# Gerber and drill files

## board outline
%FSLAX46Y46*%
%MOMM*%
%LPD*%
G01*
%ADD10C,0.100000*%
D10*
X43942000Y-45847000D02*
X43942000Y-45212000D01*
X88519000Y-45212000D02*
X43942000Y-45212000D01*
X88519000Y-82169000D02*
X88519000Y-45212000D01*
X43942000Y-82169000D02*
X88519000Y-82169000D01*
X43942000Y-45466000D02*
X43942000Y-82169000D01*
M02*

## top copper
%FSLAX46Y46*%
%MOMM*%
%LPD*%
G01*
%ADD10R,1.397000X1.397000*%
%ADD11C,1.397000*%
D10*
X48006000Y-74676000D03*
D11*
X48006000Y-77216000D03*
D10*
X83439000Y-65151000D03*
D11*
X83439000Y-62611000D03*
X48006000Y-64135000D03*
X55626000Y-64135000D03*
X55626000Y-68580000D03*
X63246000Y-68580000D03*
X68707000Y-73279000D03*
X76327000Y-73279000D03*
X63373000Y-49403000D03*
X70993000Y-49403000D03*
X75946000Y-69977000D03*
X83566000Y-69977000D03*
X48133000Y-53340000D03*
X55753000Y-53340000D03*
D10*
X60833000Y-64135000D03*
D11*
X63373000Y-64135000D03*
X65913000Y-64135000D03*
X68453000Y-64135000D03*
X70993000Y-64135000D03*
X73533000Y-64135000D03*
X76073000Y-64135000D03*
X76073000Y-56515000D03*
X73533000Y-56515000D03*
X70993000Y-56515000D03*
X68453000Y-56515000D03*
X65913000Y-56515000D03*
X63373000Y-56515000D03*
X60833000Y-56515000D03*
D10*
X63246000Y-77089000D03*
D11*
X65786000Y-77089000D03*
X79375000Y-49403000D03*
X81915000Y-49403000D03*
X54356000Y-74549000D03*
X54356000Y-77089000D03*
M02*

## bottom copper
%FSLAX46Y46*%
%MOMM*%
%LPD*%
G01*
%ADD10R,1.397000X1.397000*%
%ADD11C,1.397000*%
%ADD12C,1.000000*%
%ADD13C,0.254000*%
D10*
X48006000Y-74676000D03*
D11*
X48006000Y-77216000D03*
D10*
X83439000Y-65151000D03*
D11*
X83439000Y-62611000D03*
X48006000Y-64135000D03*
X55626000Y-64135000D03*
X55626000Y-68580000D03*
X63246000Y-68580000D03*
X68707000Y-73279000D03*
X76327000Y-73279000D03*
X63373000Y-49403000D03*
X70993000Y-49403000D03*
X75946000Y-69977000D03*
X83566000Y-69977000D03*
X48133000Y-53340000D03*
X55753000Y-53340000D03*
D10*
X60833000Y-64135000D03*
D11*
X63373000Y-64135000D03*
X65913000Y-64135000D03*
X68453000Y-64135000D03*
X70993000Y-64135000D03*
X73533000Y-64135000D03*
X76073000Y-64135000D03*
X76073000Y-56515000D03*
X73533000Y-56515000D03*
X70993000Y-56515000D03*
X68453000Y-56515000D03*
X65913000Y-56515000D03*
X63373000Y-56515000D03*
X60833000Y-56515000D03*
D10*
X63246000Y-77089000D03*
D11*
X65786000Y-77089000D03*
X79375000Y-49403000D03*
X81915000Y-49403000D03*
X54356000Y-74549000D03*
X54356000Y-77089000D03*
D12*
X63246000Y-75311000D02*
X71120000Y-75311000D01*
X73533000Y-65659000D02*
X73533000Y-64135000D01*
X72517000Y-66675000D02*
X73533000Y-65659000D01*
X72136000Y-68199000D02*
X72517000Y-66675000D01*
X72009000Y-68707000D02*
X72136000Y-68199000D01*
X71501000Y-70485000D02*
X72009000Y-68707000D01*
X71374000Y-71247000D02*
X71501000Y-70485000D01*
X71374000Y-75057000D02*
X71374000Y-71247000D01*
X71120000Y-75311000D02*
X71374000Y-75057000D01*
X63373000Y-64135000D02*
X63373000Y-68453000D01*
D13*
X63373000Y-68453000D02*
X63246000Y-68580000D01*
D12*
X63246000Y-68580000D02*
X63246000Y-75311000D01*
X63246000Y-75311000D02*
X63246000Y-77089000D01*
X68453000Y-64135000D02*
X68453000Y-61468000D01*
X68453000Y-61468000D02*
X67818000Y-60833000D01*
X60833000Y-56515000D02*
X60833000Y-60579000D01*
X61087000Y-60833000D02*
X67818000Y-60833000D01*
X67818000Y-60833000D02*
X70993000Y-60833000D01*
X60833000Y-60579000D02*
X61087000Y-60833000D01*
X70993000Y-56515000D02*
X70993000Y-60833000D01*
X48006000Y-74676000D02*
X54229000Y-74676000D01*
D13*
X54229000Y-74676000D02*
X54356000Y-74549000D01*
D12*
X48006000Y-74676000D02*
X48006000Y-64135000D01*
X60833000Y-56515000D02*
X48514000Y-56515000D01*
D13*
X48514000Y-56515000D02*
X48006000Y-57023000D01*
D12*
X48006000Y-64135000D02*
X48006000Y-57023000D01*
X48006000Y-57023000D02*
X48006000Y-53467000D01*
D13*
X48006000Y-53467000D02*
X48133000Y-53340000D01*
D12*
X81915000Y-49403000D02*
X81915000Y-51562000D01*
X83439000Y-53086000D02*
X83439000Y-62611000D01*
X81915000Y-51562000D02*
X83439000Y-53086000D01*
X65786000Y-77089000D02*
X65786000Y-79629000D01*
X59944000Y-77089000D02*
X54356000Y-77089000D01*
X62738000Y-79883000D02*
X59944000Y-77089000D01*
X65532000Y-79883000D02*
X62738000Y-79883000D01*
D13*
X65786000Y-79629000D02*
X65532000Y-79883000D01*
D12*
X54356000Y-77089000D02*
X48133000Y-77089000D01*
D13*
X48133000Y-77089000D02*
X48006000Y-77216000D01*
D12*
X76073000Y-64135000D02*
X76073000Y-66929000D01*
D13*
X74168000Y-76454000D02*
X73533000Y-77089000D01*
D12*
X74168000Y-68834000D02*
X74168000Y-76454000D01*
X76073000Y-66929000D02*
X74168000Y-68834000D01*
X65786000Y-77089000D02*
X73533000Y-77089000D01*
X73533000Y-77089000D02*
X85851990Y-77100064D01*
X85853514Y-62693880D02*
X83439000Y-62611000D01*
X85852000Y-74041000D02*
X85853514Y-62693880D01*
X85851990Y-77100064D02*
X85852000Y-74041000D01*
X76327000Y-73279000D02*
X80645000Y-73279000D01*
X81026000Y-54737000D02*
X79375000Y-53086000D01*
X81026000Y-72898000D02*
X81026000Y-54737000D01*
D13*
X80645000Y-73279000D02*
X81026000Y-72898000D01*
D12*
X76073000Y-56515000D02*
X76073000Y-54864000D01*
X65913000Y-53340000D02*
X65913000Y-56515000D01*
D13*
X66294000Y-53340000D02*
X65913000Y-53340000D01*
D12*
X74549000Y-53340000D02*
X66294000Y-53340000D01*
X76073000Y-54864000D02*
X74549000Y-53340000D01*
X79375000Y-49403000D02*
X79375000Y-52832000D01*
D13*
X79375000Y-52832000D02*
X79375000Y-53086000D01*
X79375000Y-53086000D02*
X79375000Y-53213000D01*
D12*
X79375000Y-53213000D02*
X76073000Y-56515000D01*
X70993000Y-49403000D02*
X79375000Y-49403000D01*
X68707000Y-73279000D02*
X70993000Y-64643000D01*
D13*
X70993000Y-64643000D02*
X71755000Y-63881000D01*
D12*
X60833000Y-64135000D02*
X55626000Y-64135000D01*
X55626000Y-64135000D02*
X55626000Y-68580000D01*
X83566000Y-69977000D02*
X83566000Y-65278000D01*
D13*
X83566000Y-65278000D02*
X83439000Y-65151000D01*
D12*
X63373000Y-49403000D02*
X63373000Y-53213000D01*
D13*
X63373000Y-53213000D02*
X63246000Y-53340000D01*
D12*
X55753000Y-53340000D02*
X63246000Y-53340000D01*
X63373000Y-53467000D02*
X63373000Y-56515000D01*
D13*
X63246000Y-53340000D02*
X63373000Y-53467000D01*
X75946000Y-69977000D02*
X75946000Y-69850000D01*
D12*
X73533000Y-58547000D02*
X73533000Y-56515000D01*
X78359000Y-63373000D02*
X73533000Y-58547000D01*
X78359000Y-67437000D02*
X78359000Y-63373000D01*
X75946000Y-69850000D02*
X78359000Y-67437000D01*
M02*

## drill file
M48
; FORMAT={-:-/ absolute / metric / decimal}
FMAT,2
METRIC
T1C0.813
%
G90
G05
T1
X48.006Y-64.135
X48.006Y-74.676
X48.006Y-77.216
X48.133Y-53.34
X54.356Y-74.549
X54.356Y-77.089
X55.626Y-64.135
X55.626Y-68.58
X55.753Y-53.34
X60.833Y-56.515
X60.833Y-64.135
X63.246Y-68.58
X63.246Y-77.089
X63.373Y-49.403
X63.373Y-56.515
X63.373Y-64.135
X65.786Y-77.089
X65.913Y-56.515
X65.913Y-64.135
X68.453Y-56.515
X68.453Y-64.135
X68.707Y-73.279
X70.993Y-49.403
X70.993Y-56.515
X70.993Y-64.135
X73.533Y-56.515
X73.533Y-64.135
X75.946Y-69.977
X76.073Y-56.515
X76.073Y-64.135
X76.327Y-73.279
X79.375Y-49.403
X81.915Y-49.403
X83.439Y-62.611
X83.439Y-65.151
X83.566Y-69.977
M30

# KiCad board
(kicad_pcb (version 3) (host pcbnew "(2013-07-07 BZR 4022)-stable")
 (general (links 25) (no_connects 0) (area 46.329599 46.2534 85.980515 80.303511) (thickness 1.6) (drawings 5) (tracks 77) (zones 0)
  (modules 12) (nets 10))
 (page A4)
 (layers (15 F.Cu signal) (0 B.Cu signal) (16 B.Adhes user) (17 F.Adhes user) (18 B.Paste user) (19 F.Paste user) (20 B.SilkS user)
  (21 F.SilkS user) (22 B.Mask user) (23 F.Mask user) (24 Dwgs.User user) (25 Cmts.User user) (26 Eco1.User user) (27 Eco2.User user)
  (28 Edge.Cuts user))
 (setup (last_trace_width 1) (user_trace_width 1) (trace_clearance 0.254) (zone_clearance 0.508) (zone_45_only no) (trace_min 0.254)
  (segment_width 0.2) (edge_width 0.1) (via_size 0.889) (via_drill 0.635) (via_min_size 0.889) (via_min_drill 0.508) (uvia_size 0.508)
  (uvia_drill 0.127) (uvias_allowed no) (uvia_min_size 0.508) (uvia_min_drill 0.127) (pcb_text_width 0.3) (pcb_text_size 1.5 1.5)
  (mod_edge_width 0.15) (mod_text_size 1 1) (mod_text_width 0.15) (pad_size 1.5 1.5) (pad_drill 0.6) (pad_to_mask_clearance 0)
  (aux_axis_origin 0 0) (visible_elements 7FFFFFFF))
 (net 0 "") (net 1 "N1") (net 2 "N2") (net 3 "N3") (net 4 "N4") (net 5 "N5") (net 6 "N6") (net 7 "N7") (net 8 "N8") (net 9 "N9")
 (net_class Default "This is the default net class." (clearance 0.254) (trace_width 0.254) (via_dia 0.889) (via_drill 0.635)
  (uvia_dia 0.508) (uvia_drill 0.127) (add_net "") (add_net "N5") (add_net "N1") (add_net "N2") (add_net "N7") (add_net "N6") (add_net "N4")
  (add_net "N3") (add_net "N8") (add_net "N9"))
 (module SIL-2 (layer F.Cu) (at 48.006 75.946 270)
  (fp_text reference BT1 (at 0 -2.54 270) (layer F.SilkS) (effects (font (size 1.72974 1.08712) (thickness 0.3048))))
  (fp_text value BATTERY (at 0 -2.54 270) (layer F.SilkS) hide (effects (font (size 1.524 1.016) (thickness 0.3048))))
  (pad 1 thru_hole rect (at -1.27 0 270) (size 1.397 1.397) (drill 0.8128) (layers *.Cu *.Mask F.SilkS) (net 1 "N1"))
  (pad 2 thru_hole circle (at 1.27 0 270) (size 1.397 1.397) (drill 0.8128) (layers *.Cu *.Mask F.SilkS) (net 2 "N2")))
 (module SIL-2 (layer F.Cu) (at 83.439 63.881 90)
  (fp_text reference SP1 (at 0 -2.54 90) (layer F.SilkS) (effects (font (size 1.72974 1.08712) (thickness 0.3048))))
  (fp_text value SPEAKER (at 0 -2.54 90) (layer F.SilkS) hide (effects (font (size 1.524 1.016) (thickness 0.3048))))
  (pad 1 thru_hole rect (at -1.27 0 90) (size 1.397 1.397) (drill 0.8128) (layers *.Cu *.Mask F.SilkS) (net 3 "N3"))
  (pad 2 thru_hole circle (at 1.27 0 90) (size 1.397 1.397) (drill 0.8128) (layers *.Cu *.Mask F.SilkS) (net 2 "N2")))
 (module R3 (layer F.Cu) (at 51.816 64.135) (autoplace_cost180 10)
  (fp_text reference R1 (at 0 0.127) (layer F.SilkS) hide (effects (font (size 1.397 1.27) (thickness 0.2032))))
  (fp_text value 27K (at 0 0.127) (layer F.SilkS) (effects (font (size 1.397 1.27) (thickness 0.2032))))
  (pad 1 thru_hole circle (at -3.81 0) (size 1.397 1.397) (drill 0.8128) (layers *.Cu *.Mask F.SilkS) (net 1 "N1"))
  (pad 2 thru_hole circle (at 3.81 0) (size 1.397 1.397) (drill 0.8128) (layers *.Cu *.Mask F.SilkS) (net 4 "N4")))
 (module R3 (layer F.Cu) (at 59.436 68.58) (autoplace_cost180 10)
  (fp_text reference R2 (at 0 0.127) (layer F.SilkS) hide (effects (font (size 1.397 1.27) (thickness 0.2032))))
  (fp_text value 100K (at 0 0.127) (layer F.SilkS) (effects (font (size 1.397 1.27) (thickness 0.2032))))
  (pad 1 thru_hole circle (at -3.81 0) (size 1.397 1.397) (drill 0.8128) (layers *.Cu *.Mask F.SilkS) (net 4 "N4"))
  (pad 2 thru_hole circle (at 3.81 0) (size 1.397 1.397) (drill 0.8128) (layers *.Cu *.Mask F.SilkS) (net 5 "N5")))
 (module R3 (layer F.Cu) (at 72.517 73.279) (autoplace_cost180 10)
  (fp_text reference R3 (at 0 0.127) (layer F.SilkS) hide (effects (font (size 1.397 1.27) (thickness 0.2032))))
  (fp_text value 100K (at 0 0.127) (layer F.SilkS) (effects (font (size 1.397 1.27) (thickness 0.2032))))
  (pad 1 thru_hole circle (at -3.81 0) (size 1.397 1.397) (drill 0.8128) (layers *.Cu *.Mask F.SilkS) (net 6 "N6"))
  (pad 2 thru_hole circle (at 3.81 0) (size 1.397 1.397) (drill 0.8128) (layers *.Cu *.Mask F.SilkS) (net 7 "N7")))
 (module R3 (layer F.Cu) (at 67.183 49.403) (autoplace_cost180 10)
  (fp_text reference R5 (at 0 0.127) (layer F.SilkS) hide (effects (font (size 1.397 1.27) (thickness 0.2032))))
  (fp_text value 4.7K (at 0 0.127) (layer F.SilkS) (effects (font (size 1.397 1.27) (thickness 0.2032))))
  (pad 1 thru_hole circle (at -3.81 0) (size 1.397 1.397) (drill 0.8128) (layers *.Cu *.Mask F.SilkS) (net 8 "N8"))
  (pad 2 thru_hole circle (at 3.81 0) (size 1.397 1.397) (drill 0.8128) (layers *.Cu *.Mask F.SilkS) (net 7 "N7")))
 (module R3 (layer F.Cu) (at 79.756 69.977) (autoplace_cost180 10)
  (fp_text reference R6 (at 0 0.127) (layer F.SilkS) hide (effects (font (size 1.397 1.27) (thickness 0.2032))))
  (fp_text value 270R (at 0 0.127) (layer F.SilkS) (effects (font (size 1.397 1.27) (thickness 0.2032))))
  (pad 1 thru_hole circle (at -3.81 0) (size 1.397 1.397) (drill 0.8128) (layers *.Cu *.Mask F.SilkS) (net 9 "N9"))
  (pad 2 thru_hole circle (at 3.81 0) (size 1.397 1.397) (drill 0.8128) (layers *.Cu *.Mask F.SilkS) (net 3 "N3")))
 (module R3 (layer F.Cu) (at 51.943 53.34) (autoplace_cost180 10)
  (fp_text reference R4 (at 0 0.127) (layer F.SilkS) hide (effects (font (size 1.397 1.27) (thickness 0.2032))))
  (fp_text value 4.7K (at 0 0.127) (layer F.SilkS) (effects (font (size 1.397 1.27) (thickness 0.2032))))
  (pad 1 thru_hole circle (at -3.81 0) (size 1.397 1.397) (drill 0.8128) (layers *.Cu *.Mask F.SilkS) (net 1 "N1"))
  (pad 2 thru_hole circle (at 3.81 0) (size 1.397 1.397) (drill 0.8128) (layers *.Cu *.Mask F.SilkS) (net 8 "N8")))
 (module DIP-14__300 (layer F.Cu) (at 68.453 60.325)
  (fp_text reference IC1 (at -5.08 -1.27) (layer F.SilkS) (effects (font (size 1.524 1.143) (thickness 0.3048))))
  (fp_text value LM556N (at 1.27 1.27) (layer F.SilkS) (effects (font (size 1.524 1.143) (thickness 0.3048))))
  (pad 1 thru_hole rect (at -7.62 3.81) (size 1.397 1.397) (drill 0.8128) (layers *.Cu *.Mask F.SilkS) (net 4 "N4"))
  (pad 2 thru_hole circle (at -5.08 3.81) (size 1.397 1.397) (drill 0.8128) (layers *.Cu *.Mask F.SilkS) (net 5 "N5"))
  (pad 3 thru_hole circle (at -2.54 3.81) (size 1.397 1.397) (drill 0.8128) (layers *.Cu *.Mask F.SilkS))
  (pad 4 thru_hole circle (at 0 3.81) (size 1.397 1.397) (drill 0.8128) (layers *.Cu *.Mask F.SilkS) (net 1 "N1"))
  (pad 5 thru_hole circle (at 2.54 3.81) (size 1.397 1.397) (drill 0.8128) (layers *.Cu *.Mask F.SilkS) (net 6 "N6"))
  (pad 6 thru_hole circle (at 5.08 3.81) (size 1.397 1.397) (drill 0.8128) (layers *.Cu *.Mask F.SilkS) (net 5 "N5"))
  (pad 7 thru_hole circle (at 7.62 3.81) (size 1.397 1.397) (drill 0.8128) (layers *.Cu *.Mask F.SilkS) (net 2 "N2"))
  (pad 8 thru_hole circle (at 7.62 -3.81) (size 1.397 1.397) (drill 0.8128) (layers *.Cu *.Mask F.SilkS) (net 7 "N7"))
  (pad 9 thru_hole circle (at 5.08 -3.81) (size 1.397 1.397) (drill 0.8128) (layers *.Cu *.Mask F.SilkS) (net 9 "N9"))
  (pad 10 thru_hole circle (at 2.54 -3.81) (size 1.397 1.397) (drill 0.8128) (layers *.Cu *.Mask F.SilkS) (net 1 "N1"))
  (pad 11 thru_hole circle (at 0 -3.81) (size 1.397 1.397) (drill 0.8128) (layers *.Cu *.Mask F.SilkS))
  (pad 12 thru_hole circle (at -2.54 -3.81) (size 1.397 1.397) (drill 0.8128) (layers *.Cu *.Mask F.SilkS) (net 7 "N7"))
  (pad 13 thru_hole circle (at -5.08 -3.81) (size 1.397 1.397) (drill 0.8128) (layers *.Cu *.Mask F.SilkS) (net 8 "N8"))
  (pad 14 thru_hole circle (at -7.62 -3.81) (size 1.397 1.397) (drill 0.8128) (layers *.Cu *.Mask F.SilkS) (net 1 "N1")))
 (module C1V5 (layer F.Cu) (at 64.516 77.089)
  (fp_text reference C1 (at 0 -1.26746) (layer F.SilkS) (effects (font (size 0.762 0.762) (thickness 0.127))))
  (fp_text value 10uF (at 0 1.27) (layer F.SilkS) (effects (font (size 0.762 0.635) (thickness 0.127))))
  (pad 1 thru_hole rect (at -1.27 0) (size 1.397 1.397) (drill 0.8128) (layers *.Cu *.Mask F.SilkS) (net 5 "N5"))
  (pad 2 thru_hole circle (at 1.27 0) (size 1.397 1.397) (drill 0.8128) (layers *.Cu *.Mask F.SilkS) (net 2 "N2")))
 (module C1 (layer F.Cu) (at 80.645 49.403)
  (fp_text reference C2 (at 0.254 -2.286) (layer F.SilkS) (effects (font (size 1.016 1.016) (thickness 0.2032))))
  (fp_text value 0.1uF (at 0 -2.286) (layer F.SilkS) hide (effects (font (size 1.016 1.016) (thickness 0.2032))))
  (pad 1 thru_hole circle (at -1.27 0) (size 1.397 1.397) (drill 0.8128) (layers *.Cu *.Mask F.SilkS) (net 7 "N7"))
  (pad 2 thru_hole circle (at 1.27 0) (size 1.397 1.397) (drill 0.8128) (layers *.Cu *.Mask F.SilkS) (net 2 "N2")))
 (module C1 (layer F.Cu) (at 54.356 75.819 270)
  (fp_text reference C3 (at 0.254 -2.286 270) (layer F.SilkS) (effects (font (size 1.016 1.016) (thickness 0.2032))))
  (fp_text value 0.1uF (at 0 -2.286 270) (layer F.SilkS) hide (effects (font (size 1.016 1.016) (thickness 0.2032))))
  (pad 1 thru_hole circle (at -1.27 0 270) (size 1.397 1.397) (drill 0.8128) (layers *.Cu *.Mask F.SilkS) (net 1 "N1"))
  (pad 2 thru_hole circle (at 1.27 0 270) (size 1.397 1.397) (drill 0.8128) (layers *.Cu *.Mask F.SilkS) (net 2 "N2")))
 (gr_line (start 43.942 45.847) (end 43.942 45.212) (angle 90) (layer Edge.Cuts) (width 0.1))
 (gr_line (start 88.519 45.212) (end 43.942 45.212) (angle 90) (layer Edge.Cuts) (width 0.1))
 (gr_line (start 88.519 82.169) (end 88.519 45.212) (angle 90) (layer Edge.Cuts) (width 0.1))
 (gr_line (start 43.942 82.169) (end 88.519 82.169) (angle 90) (layer Edge.Cuts) (width 0.1))
 (gr_line (start 43.942 45.466) (end 43.942 82.169) (angle 90) (layer Edge.Cuts) (width 0.1))
 (segment (start 63.246 75.311) (end 71.12 75.311) (width 1) (layer B.Cu) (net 5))
 (segment (start 73.533 65.659) (end 73.533 64.135) (width 1) (layer B.Cu) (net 5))
 (segment (start 72.517 66.675) (end 73.533 65.659) (width 1) (layer B.Cu) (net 5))
 (segment (start 72.136 68.199) (end 72.517 66.675) (width 1) (layer B.Cu) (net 5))
 (segment (start 72.009 68.707) (end 72.136 68.199) (width 1) (layer B.Cu) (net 5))
 (segment (start 71.501 70.485) (end 72.009 68.707) (width 1) (layer B.Cu) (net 5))
 (segment (start 71.374 71.247) (end 71.501 70.485) (width 1) (layer B.Cu) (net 5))
 (segment (start 71.374 75.057) (end 71.374 71.247) (width 1) (layer B.Cu) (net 5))
 (segment (start 71.12 75.311) (end 71.374 75.057) (width 1) (layer B.Cu) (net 5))
 (segment (start 63.373 64.135) (end 63.373 68.453) (width 1) (layer B.Cu) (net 5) (status 20))
 (segment (start 63.373 68.453) (end 63.246 68.58) (width 0.254) (layer B.Cu) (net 5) (status 30))
 (segment (start 63.246 68.58) (end 63.246 75.311) (width 1) (layer B.Cu) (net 5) (status 10))
 (segment (start 63.246 75.311) (end 63.246 77.089) (width 1) (layer B.Cu) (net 5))
 (segment (start 68.453 64.135) (end 68.453 61.468) (width 1) (layer B.Cu) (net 1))
 (segment (start 68.453 61.468) (end 67.818 60.833) (width 1) (layer B.Cu) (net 1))
 (segment (start 60.833 56.515) (end 60.833 60.579) (width 1) (layer B.Cu) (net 1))
 (segment (start 61.087 60.833) (end 67.818 60.833) (width 1) (layer B.Cu) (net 1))
 (segment (start 67.818 60.833) (end 70.993 60.833) (width 1) (layer B.Cu) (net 1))
 (segment (start 60.833 60.579) (end 61.087 60.833) (width 1) (layer B.Cu) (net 1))
 (segment (start 70.993 56.515) (end 70.993 60.833) (width 1) (layer B.Cu) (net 1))
 (segment (start 48.006 74.676) (end 54.229 74.676) (width 1) (layer B.Cu) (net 1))
 (segment (start 54.229 74.676) (end 54.356 74.549) (width 0.254) (layer B.Cu) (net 1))
 (segment (start 48.006 74.676) (end 48.006 64.135) (width 1) (layer B.Cu) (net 1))
 (segment (start 60.833 56.515) (end 48.514 56.515) (width 1) (layer B.Cu) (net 1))
 (segment (start 48.514 56.515) (end 48.006 57.023) (width 0.254) (layer B.Cu) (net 1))
 (segment (start 48.006 64.135) (end 48.006 57.023) (width 1) (layer B.Cu) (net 1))
 (segment (start 48.006 57.023) (end 48.006 53.467) (width 1) (layer B.Cu) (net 1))
 (segment (start 48.006 53.467) (end 48.133 53.34) (width 0.254) (layer B.Cu) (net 1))
 (segment (start 81.915 49.403) (end 81.915 51.562) (width 1) (layer B.Cu) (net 2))
 (segment (start 83.439 53.086) (end 83.439 62.611) (width 1) (layer B.Cu) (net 2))
 (segment (start 81.915 51.562) (end 83.439 53.086) (width 1) (layer B.Cu) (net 2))
 (segment (start 65.786 77.089) (end 65.786 79.629) (width 1) (layer B.Cu) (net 2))
 (segment (start 59.944 77.089) (end 54.356 77.089) (width 1) (layer B.Cu) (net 2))
 (segment (start 62.738 79.883) (end 59.944 77.089) (width 1) (layer B.Cu) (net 2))
 (segment (start 65.532 79.883) (end 62.738 79.883) (width 1) (layer B.Cu) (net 2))
 (segment (start 65.786 79.629) (end 65.532 79.883) (width 0.254) (layer B.Cu) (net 2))
 (segment (start 54.356 77.089) (end 48.133 77.089) (width 1) (layer B.Cu) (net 2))
 (segment (start 48.133 77.089) (end 48.006 77.216) (width 0.254) (layer B.Cu) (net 2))
 (segment (start 76.073 64.135) (end 76.073 66.929) (width 1) (layer B.Cu) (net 2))
 (segment (start 74.168 76.454) (end 73.533 77.089) (width 0.254) (layer B.Cu) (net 2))
 (segment (start 74.168 68.834) (end 74.168 76.454) (width 1) (layer B.Cu) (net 2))
 (segment (start 76.073 66.929) (end 74.168 68.834) (width 1) (layer B.Cu) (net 2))
 (segment (start 65.786 77.089) (end 73.533 77.089) (width 1) (layer B.Cu) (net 2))
 (segment (start 73.533 77.089) (end 85.85199 77.100064) (width 1) (layer B.Cu) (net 2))
 (segment (start 85.853514 62.69388) (end 83.439 62.611) (width 1) (layer B.Cu) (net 2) (status 20))
 (segment (start 85.852 74.041) (end 85.853514 62.69388) (width 1) (layer B.Cu) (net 2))
 (segment (start 85.85199 77.100064) (end 85.852 74.041) (width 1) (layer B.Cu) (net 2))
 (segment (start 76.327 73.279) (end 80.645 73.279) (width 1) (layer B.Cu) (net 7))
 (segment (start 81.026 54.737) (end 79.375 53.086) (width 1) (layer B.Cu) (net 7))
 (segment (start 81.026 72.898) (end 81.026 54.737) (width 1) (layer B.Cu) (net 7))
 (segment (start 80.645 73.279) (end 81.026 72.898) (width 0.254) (layer B.Cu) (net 7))
 (segment (start 76.073 56.515) (end 76.073 54.864) (width 1) (layer B.Cu) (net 7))
 (segment (start 65.913 53.34) (end 65.913 56.515) (width 1) (layer B.Cu) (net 7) (status 800000))
 (segment (start 66.294 53.34) (end 65.913 53.34) (width 0.254) (layer B.Cu) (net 7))
 (segment (start 74.549 53.34) (end 66.294 53.34) (width 1) (layer B.Cu) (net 7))
 (segment (start 76.073 54.864) (end 74.549 53.34) (width 1) (layer B.Cu) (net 7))
 (segment (start 79.375 49.403) (end 79.375 52.832) (width 1) (layer B.Cu) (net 7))
 (segment (start 79.375 52.832) (end 79.375 53.086) (width 0.254) (layer B.Cu) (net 7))
 (segment (start 79.375 53.086) (end 79.375 53.213) (width 0.254) (layer B.Cu) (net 7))
 (segment (start 79.375 53.213) (end 76.073 56.515) (width 1) (layer B.Cu) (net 7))
 (segment (start 70.993 49.403) (end 79.375 49.403) (width 1) (layer B.Cu) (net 7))
 (segment (start 68.707 73.279) (end 70.993 64.643) (width 1) (layer B.Cu) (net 6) (status 10))
 (segment (start 70.993 64.643) (end 71.755 63.881) (width 0.254) (layer B.Cu) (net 6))
 (segment (start 60.833 64.135) (end 55.626 64.135) (width 1) (layer B.Cu) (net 4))
 (segment (start 55.626 64.135) (end 55.626 68.58) (width 1) (layer B.Cu) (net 4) (status 20))
 (segment (start 83.566 69.977) (end 83.566 65.278) (width 1) (layer B.Cu) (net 3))
 (segment (start 83.566 65.278) (end 83.439 65.151) (width 0.254) (layer B.Cu) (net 3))
 (segment (start 63.373 49.403) (end 63.373 53.213) (width 1) (layer B.Cu) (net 8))
 (segment (start 63.373 53.213) (end 63.246 53.34) (width 0.254) (layer B.Cu) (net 8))
 (segment (start 55.753 53.34) (end 63.246 53.34) (width 1) (layer B.Cu) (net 8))
 (segment (start 63.373 53.467) (end 63.373 56.515) (width 1) (layer B.Cu) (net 8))
 (segment (start 63.246 53.34) (end 63.373 53.467) (width 0.254) (layer B.Cu) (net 8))
 (segment (start 75.946 69.977) (end 75.946 69.85) (width 0.254) (layer B.Cu) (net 9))
 (segment (start 73.533 58.547) (end 73.533 56.515) (width 1) (layer B.Cu) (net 9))
 (segment (start 78.359 63.373) (end 73.533 58.547) (width 1) (layer B.Cu) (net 9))
 (segment (start 78.359 67.437) (end 78.359 63.373) (width 1) (layer B.Cu) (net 9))
 (segment (start 75.946 69.85) (end 78.359 67.437) (width 1) (layer B.Cu) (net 9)))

